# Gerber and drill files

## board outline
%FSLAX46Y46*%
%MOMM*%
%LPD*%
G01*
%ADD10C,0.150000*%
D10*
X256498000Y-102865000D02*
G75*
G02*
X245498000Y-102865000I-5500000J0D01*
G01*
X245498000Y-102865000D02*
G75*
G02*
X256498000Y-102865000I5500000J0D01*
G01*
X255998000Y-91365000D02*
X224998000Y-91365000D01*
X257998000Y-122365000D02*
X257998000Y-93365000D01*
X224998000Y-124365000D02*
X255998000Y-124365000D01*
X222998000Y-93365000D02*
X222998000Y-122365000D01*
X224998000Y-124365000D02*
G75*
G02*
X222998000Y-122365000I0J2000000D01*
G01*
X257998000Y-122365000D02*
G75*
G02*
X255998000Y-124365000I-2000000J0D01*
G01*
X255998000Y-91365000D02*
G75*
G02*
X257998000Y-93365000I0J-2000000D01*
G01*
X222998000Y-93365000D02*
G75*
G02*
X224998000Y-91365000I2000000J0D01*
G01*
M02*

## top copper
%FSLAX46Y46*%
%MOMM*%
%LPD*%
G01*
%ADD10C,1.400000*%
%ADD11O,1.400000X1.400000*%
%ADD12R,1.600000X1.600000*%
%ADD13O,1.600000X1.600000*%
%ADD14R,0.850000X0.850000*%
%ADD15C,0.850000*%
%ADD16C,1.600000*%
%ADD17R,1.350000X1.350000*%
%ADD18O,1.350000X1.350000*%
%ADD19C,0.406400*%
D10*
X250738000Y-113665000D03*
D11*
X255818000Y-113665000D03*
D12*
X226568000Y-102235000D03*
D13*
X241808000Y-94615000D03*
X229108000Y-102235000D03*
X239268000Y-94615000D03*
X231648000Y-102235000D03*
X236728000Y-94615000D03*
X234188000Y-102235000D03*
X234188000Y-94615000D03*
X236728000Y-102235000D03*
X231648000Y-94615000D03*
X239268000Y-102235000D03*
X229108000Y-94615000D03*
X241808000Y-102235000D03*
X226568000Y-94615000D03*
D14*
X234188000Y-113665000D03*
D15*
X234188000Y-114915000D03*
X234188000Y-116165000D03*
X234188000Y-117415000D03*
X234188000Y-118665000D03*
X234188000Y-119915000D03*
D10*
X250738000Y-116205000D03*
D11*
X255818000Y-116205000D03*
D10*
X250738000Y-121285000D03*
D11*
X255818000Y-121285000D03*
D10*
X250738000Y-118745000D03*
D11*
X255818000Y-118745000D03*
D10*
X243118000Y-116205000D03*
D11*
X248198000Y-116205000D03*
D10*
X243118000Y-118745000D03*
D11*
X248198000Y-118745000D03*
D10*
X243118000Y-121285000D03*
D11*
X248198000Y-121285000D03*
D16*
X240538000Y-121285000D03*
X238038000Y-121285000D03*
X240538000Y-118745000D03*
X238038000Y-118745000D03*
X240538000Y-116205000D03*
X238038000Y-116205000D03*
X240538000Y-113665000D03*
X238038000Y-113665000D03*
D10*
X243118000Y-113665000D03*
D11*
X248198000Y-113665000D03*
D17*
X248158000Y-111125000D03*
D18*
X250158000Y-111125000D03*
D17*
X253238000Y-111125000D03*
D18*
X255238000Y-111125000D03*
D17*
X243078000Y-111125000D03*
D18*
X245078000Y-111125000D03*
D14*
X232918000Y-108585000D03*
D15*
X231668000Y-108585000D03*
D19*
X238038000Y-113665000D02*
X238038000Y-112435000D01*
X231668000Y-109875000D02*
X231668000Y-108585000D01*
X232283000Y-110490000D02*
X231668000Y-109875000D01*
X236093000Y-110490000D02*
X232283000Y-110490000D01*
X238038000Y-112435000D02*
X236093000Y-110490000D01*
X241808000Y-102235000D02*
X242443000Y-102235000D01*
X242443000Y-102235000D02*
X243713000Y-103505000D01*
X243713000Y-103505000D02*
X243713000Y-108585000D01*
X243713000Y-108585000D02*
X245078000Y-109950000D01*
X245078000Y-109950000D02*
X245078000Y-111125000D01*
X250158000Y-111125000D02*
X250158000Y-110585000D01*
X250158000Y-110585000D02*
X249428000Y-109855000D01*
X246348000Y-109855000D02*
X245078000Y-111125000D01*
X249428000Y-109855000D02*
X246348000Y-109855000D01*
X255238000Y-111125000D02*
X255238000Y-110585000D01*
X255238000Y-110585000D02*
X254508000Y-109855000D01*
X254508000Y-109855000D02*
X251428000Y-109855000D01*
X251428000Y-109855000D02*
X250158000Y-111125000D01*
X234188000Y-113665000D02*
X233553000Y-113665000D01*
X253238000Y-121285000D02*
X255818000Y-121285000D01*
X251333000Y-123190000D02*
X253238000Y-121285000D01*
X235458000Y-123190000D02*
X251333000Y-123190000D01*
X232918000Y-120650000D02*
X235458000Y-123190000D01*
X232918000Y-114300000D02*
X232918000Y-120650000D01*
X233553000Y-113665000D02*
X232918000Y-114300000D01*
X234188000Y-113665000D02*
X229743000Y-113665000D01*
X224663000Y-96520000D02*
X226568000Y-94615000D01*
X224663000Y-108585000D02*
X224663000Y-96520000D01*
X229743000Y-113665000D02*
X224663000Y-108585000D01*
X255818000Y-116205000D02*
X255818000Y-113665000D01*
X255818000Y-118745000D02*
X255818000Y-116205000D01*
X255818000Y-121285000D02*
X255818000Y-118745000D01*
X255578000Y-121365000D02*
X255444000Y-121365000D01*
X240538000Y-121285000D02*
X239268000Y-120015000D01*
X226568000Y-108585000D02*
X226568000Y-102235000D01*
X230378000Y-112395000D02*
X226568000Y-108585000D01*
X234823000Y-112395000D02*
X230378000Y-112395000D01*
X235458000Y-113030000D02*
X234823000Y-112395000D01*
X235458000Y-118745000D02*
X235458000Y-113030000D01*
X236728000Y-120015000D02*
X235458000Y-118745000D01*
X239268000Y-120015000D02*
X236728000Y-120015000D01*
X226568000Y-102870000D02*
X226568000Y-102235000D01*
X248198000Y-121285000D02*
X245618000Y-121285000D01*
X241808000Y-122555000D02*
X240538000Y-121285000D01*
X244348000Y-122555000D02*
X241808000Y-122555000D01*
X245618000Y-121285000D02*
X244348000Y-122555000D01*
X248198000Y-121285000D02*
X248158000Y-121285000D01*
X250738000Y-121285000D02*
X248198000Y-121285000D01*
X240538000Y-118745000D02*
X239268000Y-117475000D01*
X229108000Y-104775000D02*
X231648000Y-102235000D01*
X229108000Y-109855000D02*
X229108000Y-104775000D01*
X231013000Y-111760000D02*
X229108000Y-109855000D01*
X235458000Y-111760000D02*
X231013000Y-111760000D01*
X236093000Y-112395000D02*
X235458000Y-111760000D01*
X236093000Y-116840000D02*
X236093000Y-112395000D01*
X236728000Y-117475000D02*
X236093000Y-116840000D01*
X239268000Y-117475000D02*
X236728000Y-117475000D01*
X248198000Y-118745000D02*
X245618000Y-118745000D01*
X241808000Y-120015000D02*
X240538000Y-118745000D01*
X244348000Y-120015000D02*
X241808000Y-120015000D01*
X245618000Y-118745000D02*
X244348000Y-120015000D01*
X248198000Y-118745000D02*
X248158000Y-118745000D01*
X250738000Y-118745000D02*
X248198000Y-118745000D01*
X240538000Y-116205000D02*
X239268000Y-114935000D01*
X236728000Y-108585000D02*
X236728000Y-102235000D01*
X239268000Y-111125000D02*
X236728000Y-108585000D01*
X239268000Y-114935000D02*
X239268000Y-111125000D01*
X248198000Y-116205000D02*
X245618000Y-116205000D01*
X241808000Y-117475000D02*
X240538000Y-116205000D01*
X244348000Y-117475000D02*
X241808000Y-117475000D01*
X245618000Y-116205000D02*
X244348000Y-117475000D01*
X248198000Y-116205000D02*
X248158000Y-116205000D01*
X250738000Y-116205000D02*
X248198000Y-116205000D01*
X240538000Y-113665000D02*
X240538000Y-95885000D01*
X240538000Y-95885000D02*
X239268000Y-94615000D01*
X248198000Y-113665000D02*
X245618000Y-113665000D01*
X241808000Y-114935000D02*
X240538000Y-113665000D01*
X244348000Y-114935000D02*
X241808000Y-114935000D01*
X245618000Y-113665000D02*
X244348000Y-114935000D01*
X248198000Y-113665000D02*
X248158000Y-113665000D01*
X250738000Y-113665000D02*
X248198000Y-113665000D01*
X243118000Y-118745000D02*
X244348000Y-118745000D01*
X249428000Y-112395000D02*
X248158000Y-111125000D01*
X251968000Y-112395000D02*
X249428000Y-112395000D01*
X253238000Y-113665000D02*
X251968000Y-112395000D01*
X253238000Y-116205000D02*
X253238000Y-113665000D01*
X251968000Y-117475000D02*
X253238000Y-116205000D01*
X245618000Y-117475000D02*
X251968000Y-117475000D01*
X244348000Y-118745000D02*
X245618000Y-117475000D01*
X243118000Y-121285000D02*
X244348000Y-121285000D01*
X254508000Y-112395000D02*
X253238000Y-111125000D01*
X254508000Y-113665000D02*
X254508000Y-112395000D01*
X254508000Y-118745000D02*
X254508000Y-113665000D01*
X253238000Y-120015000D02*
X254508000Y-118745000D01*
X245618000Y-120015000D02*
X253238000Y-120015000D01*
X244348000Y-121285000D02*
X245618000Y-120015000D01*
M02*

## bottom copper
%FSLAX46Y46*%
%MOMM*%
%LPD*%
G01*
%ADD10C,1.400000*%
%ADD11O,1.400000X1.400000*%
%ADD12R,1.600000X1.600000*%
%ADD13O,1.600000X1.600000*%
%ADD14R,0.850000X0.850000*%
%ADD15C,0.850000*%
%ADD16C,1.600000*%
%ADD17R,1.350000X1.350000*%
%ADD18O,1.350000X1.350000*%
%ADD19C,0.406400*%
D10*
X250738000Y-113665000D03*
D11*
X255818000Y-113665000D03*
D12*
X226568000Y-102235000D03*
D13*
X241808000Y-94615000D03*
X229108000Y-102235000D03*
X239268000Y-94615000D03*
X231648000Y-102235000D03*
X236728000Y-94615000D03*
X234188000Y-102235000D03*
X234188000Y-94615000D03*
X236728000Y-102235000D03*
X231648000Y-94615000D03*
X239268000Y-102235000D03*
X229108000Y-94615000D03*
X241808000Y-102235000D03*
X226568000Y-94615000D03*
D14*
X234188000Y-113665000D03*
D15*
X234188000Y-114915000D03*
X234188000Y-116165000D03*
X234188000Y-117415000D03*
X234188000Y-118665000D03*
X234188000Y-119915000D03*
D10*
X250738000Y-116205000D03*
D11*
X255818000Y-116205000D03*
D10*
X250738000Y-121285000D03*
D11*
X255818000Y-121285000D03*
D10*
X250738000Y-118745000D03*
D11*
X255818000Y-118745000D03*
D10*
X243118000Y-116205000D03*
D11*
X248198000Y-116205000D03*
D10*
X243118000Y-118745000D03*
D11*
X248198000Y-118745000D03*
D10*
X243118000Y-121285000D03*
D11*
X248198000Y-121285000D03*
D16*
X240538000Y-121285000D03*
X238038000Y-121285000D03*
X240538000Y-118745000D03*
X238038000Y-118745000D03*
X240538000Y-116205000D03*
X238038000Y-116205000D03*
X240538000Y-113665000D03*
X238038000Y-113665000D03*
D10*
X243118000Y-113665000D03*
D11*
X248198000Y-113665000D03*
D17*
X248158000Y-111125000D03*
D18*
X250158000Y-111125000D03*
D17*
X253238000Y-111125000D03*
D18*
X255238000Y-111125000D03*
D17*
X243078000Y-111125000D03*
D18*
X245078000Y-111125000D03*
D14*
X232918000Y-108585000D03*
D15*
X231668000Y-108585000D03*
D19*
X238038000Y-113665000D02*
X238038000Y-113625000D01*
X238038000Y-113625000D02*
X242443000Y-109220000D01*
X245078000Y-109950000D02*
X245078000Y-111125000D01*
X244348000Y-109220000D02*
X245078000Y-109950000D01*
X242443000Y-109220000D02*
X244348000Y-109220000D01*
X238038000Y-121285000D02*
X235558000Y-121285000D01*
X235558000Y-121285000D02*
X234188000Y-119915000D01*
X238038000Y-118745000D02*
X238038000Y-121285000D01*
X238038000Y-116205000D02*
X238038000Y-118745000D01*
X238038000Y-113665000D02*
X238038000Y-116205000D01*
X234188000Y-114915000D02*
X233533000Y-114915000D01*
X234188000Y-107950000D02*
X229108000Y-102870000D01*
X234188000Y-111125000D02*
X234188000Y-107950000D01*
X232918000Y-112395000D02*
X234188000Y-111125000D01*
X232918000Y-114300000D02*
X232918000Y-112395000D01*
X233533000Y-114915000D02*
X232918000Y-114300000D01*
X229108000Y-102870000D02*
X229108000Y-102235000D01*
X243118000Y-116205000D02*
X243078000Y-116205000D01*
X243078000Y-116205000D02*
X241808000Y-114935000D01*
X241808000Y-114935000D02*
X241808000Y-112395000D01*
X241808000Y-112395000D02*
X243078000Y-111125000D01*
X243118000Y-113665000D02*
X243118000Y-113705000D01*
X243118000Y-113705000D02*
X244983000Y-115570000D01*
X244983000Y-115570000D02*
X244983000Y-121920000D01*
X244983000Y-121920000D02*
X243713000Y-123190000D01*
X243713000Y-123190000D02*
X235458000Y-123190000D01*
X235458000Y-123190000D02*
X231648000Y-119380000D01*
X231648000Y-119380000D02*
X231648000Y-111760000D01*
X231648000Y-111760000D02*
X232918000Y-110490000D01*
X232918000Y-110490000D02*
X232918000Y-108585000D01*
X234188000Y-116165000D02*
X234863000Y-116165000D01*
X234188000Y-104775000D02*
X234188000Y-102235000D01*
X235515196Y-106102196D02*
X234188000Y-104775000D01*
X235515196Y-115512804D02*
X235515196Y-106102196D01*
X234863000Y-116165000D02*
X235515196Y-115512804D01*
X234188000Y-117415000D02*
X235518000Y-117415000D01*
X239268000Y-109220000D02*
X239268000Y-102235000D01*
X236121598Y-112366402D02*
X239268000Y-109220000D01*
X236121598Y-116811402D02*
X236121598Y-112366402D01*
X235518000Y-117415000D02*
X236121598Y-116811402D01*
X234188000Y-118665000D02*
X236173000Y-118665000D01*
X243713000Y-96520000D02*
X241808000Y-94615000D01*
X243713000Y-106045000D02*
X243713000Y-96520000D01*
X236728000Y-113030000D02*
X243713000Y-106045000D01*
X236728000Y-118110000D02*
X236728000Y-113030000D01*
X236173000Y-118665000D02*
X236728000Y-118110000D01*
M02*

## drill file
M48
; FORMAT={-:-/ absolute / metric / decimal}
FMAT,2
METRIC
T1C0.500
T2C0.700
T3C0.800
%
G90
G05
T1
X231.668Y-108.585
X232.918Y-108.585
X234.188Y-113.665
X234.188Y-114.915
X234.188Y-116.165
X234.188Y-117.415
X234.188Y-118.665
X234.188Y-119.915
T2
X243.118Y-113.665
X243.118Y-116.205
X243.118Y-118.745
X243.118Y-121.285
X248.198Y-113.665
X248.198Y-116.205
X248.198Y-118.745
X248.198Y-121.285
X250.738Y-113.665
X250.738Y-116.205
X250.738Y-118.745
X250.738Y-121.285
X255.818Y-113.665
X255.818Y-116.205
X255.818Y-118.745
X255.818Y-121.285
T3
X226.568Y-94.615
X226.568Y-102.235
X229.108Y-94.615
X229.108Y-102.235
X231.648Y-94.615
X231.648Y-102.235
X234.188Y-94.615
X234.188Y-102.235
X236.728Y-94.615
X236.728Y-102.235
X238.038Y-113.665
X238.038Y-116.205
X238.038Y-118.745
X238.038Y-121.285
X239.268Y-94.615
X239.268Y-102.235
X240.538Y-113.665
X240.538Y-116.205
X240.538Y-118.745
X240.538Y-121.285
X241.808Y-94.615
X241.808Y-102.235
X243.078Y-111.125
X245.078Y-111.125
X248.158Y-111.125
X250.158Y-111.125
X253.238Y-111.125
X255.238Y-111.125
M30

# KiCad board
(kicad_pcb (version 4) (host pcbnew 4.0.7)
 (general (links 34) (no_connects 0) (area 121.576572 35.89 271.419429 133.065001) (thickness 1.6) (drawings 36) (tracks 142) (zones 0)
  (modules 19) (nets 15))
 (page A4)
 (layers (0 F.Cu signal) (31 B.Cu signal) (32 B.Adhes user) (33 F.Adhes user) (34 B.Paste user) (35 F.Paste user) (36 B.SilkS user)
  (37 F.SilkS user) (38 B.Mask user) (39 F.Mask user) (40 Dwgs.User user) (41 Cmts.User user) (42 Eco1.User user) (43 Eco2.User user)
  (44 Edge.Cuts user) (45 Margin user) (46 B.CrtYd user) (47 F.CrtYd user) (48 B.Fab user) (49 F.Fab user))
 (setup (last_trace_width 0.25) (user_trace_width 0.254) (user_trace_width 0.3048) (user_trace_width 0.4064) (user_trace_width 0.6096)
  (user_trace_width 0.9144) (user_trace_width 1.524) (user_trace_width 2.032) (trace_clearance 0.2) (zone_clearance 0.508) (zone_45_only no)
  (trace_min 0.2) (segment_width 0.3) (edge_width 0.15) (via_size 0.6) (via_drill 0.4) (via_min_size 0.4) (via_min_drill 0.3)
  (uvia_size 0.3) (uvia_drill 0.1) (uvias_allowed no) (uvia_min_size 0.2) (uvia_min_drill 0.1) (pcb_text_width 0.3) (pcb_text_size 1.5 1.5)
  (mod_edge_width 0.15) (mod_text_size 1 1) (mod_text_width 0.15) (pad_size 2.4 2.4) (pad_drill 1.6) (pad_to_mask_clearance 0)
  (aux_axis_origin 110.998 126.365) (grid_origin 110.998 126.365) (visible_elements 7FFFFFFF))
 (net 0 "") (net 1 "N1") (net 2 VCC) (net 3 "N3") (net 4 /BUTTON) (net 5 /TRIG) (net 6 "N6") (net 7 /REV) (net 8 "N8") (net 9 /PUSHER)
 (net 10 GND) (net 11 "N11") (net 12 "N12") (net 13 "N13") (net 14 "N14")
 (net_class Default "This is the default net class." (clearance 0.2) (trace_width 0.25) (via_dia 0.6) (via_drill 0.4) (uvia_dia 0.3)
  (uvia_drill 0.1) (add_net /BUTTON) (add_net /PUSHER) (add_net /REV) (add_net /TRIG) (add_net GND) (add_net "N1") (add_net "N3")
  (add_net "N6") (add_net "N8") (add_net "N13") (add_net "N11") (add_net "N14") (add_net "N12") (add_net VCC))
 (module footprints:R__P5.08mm (layer F.Cu) (at 253.238 113.665)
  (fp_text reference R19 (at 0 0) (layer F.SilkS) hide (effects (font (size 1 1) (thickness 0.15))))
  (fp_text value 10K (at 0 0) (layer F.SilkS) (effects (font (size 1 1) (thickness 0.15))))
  (pad 1 thru_hole circle (at -2.5 0) (size 1.4 1.4) (drill 0.7) (layers *.Cu *.Mask) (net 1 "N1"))
  (pad 2 thru_hole oval (at 2.58 0) (size 1.4 1.4) (drill 0.7) (layers *.Cu *.Mask) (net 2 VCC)))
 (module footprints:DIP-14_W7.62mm (layer F.Cu) (at 226.568 102.235 90)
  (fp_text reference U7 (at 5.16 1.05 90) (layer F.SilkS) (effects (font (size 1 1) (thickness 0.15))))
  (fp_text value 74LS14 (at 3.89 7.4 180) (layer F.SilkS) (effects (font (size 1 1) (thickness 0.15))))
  (pad 1 thru_hole rect (at 0 0 90) (size 1.6 1.6) (drill 0.8) (layers *.Cu *.Mask) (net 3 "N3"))
  (pad 8 thru_hole oval (at 7.62 15.24 90) (size 1.6 1.6) (drill 0.8) (layers *.Cu *.Mask) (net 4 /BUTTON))
  (pad 2 thru_hole oval (at 0 2.54 90) (size 1.6 1.6) (drill 0.8) (layers *.Cu *.Mask) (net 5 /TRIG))
  (pad 9 thru_hole oval (at 7.62 12.7 90) (size 1.6 1.6) (drill 0.8) (layers *.Cu *.Mask) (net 1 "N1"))
  (pad 3 thru_hole oval (at 0 5.08 90) (size 1.6 1.6) (drill 0.8) (layers *.Cu *.Mask) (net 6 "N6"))
  (pad 10 thru_hole oval (at 7.62 10.16 90) (size 1.6 1.6) (drill 0.8) (layers *.Cu *.Mask))
  (pad 4 thru_hole oval (at 0 7.62 90) (size 1.6 1.6) (drill 0.8) (layers *.Cu *.Mask) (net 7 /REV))
  (pad 11 thru_hole oval (at 7.62 7.62 90) (size 1.6 1.6) (drill 0.8) (layers *.Cu *.Mask))
  (pad 5 thru_hole oval (at 0 10.16 90) (size 1.6 1.6) (drill 0.8) (layers *.Cu *.Mask) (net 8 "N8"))
  (pad 12 thru_hole oval (at 7.62 5.08 90) (size 1.6 1.6) (drill 0.8) (layers *.Cu *.Mask))
  (pad 6 thru_hole oval (at 0 12.7 90) (size 1.6 1.6) (drill 0.8) (layers *.Cu *.Mask) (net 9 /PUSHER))
  (pad 13 thru_hole oval (at 7.62 2.54 90) (size 1.6 1.6) (drill 0.8) (layers *.Cu *.Mask))
  (pad 7 thru_hole oval (at 0 15.24 90) (size 1.6 1.6) (drill 0.8) (layers *.Cu *.Mask) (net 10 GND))
  (pad 14 thru_hole oval (at 7.62 0 90) (size 1.6 1.6) (drill 0.8) (layers *.Cu *.Mask) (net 2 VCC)))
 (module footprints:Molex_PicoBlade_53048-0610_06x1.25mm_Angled (layer F.Cu) (at 234.188 113.665 270)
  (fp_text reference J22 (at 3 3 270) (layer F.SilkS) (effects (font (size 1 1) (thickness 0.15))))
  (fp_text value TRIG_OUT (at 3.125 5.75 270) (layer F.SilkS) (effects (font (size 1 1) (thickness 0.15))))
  (pad 1 thru_hole rect (at 0 0 270) (size 0.85 0.85) (drill 0.5) (layers *.Cu *.Mask) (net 2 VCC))
  (pad 2 thru_hole circle (at 1.25 0 270) (size 0.85 0.85) (drill 0.5) (layers *.Cu *.Mask) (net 5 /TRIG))
  (pad 3 thru_hole circle (at 2.5 0 270) (size 0.85 0.85) (drill 0.5) (layers *.Cu *.Mask) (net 7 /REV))
  (pad 4 thru_hole circle (at 3.75 0 270) (size 0.85 0.85) (drill 0.5) (layers *.Cu *.Mask) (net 9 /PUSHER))
  (pad 5 thru_hole circle (at 5 0 270) (size 0.85 0.85) (drill 0.5) (layers *.Cu *.Mask) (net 4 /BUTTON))
  (pad 6 thru_hole circle (at 6.25 0 270) (size 0.85 0.85) (drill 0.5) (layers *.Cu *.Mask) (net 10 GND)))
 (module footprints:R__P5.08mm (layer F.Cu) (at 253.238 116.205)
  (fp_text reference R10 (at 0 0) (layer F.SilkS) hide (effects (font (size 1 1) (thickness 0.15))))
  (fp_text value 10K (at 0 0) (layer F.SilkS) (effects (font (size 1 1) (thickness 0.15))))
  (pad 1 thru_hole circle (at -2.5 0) (size 1.4 1.4) (drill 0.7) (layers *.Cu *.Mask) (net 8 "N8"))
  (pad 2 thru_hole oval (at 2.58 0) (size 1.4 1.4) (drill 0.7) (layers *.Cu *.Mask) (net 2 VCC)))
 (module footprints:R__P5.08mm (layer F.Cu) (at 253.238 121.285)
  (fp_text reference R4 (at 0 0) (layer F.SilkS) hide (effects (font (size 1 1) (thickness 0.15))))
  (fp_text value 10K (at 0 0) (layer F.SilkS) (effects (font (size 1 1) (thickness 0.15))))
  (pad 1 thru_hole circle (at -2.5 0) (size 1.4 1.4) (drill 0.7) (layers *.Cu *.Mask) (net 3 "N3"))
  (pad 2 thru_hole oval (at 2.58 0) (size 1.4 1.4) (drill 0.7) (layers *.Cu *.Mask) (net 2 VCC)))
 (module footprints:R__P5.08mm (layer F.Cu) (at 253.238 118.745)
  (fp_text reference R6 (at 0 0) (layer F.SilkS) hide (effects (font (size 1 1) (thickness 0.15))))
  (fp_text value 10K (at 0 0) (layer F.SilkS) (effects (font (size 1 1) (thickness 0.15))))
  (pad 1 thru_hole circle (at -2.5 0) (size 1.4 1.4) (drill 0.7) (layers *.Cu *.Mask) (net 6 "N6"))
  (pad 2 thru_hole oval (at 2.58 0) (size 1.4 1.4) (drill 0.7) (layers *.Cu *.Mask) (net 2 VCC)))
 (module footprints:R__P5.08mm (layer F.Cu) (at 245.618 116.205)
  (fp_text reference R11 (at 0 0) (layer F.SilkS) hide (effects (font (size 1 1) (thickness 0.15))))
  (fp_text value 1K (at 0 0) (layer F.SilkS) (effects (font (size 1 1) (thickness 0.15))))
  (pad 1 thru_hole circle (at -2.5 0) (size 1.4 1.4) (drill 0.7) (layers *.Cu *.Mask) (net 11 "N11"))
  (pad 2 thru_hole oval (at 2.58 0) (size 1.4 1.4) (drill 0.7) (layers *.Cu *.Mask) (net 8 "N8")))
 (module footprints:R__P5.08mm (layer F.Cu) (at 245.618 118.745)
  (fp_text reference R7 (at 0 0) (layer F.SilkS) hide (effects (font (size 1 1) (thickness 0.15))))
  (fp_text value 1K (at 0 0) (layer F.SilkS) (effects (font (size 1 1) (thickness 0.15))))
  (pad 1 thru_hole circle (at -2.5 0) (size 1.4 1.4) (drill 0.7) (layers *.Cu *.Mask) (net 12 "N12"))
  (pad 2 thru_hole oval (at 2.58 0) (size 1.4 1.4) (drill 0.7) (layers *.Cu *.Mask) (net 6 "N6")))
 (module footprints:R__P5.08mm (layer F.Cu) (at 245.618 121.285)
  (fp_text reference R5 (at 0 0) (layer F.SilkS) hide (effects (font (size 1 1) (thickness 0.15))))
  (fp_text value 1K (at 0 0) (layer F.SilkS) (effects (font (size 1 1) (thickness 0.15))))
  (pad 1 thru_hole circle (at -2.5 0) (size 1.4 1.4) (drill 0.7) (layers *.Cu *.Mask) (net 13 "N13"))
  (pad 2 thru_hole oval (at 2.58 0) (size 1.4 1.4) (drill 0.7) (layers *.Cu *.Mask) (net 3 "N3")))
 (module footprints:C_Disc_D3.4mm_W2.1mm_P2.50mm (layer F.Cu) (at 240.538 121.285 180)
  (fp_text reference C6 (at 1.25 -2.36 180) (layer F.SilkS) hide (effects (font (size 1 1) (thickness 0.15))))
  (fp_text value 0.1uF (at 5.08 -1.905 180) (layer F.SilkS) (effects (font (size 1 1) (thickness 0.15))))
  (pad 1 thru_hole circle (at 0 0 180) (size 1.6 1.6) (drill 0.8) (layers *.Cu *.Mask) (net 3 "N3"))
  (pad 2 thru_hole circle (at 2.5 0 180) (size 1.6 1.6) (drill 0.8) (layers *.Cu *.Mask) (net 10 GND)))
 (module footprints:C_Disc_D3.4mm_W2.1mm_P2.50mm (layer F.Cu) (at 240.538 118.745 180)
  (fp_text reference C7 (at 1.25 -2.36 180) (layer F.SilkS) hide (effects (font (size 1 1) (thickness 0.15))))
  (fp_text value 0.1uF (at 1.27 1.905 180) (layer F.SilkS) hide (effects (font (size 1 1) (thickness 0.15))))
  (pad 1 thru_hole circle (at 0 0 180) (size 1.6 1.6) (drill 0.8) (layers *.Cu *.Mask) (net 6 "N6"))
  (pad 2 thru_hole circle (at 2.5 0 180) (size 1.6 1.6) (drill 0.8) (layers *.Cu *.Mask) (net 10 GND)))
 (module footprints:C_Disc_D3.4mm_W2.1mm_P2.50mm (layer F.Cu) (at 240.538 116.205 180)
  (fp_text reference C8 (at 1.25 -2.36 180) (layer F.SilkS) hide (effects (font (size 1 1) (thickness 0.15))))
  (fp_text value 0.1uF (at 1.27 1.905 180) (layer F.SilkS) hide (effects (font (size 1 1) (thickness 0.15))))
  (pad 1 thru_hole circle (at 0 0 180) (size 1.6 1.6) (drill 0.8) (layers *.Cu *.Mask) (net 8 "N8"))
  (pad 2 thru_hole circle (at 2.5 0 180) (size 1.6 1.6) (drill 0.8) (layers *.Cu *.Mask) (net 10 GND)))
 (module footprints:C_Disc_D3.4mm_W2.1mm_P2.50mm (layer F.Cu) (at 240.538 113.665 180)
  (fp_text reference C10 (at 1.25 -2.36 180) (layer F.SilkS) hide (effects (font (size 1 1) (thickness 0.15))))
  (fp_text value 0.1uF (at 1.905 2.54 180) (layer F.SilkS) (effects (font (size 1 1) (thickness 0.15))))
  (pad 1 thru_hole circle (at 0 0 180) (size 1.6 1.6) (drill 0.8) (layers *.Cu *.Mask) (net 1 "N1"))
  (pad 2 thru_hole circle (at 2.5 0 180) (size 1.6 1.6) (drill 0.8) (layers *.Cu *.Mask) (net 10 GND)))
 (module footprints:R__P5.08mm (layer F.Cu) (at 245.618 113.665)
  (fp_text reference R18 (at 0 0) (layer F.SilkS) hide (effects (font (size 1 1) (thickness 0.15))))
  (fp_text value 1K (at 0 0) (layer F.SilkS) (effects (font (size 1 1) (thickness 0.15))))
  (pad 1 thru_hole circle (at -2.5 0) (size 1.4 1.4) (drill 0.7) (layers *.Cu *.Mask) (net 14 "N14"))
  (pad 2 thru_hole oval (at 2.58 0) (size 1.4 1.4) (drill 0.7) (layers *.Cu *.Mask) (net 1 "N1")))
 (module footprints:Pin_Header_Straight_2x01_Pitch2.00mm (layer F.Cu) (at 248.158 111.125)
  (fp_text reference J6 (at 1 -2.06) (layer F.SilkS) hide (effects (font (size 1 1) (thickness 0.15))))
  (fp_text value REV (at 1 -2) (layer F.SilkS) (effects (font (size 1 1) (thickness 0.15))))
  (pad 1 thru_hole rect (at 0 0) (size 1.35 1.35) (drill 0.8) (layers *.Cu *.Mask) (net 12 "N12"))
  (pad 2 thru_hole oval (at 2 0) (size 1.35 1.35) (drill 0.8) (layers *.Cu *.Mask) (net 10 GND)))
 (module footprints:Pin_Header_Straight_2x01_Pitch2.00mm (layer F.Cu) (at 253.238 111.125)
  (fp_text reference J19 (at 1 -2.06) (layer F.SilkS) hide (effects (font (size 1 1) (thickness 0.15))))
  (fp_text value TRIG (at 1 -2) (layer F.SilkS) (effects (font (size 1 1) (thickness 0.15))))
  (pad 1 thru_hole rect (at 0 0) (size 1.35 1.35) (drill 0.8) (layers *.Cu *.Mask) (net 13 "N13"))
  (pad 2 thru_hole oval (at 2 0) (size 1.35 1.35) (drill 0.8) (layers *.Cu *.Mask) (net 10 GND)))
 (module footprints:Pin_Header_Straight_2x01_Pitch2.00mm (layer F.Cu) (at 243.078 111.125)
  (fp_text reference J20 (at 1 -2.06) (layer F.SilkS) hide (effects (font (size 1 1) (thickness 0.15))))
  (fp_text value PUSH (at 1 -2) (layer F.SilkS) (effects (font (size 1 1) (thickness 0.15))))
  (pad 1 thru_hole rect (at 0 0) (size 1.35 1.35) (drill 0.8) (layers *.Cu *.Mask) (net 11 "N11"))
  (pad 2 thru_hole oval (at 2 0) (size 1.35 1.35) (drill 0.8) (layers *.Cu *.Mask) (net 10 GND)))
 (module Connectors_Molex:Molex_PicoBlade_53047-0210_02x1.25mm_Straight (layer F.Cu) (at 232.918 108.585 180)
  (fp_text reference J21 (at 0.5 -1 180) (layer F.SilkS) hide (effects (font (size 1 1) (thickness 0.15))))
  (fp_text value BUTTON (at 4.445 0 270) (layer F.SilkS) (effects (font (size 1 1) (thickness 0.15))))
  (pad 1 thru_hole rect (at 0 0 180) (size 0.85 0.85) (drill 0.5) (layers *.Cu *.Mask) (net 14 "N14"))
  (pad 2 thru_hole circle (at 1.25 0 180) (size 0.85 0.85) (drill 0.5) (layers *.Cu *.Mask) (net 10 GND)))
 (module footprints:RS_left (layer F.Cu) (at 237.998 105.41)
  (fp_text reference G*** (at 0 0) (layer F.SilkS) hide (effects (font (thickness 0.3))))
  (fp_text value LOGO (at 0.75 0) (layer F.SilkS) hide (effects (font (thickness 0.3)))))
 (gr_circle (center 250.998 102.865) (end 245.498 102.865) (layer Edge.Cuts) (width 0.15))
 (gr_line (start 255.998 91.365) (end 224.998 91.365) (angle 90) (layer Edge.Cuts) (width 0.15))
 (gr_line (start 257.998 122.365) (end 257.998 93.365) (angle 90) (layer Edge.Cuts) (width 0.15))
 (gr_line (start 224.998 124.365) (end 255.998 124.365) (angle 90) (layer Edge.Cuts) (width 0.15))
 (gr_line (start 222.998 93.365) (end 222.998 122.365) (angle 90) (layer Edge.Cuts) (width 0.15))
 (gr_arc (start 224.998 122.365) (end 224.998 124.365) (angle 90) (layer Edge.Cuts) (width 0.15))
 (gr_arc (start 255.998 122.365) (end 257.998 122.365) (angle 90) (layer Edge.Cuts) (width 0.15))
 (gr_arc (start 255.998 93.365) (end 255.998 91.365) (angle 90) (layer Edge.Cuts) (width 0.15))
 (gr_arc (start 224.998 93.365) (end 222.998 93.365) (angle 90) (layer Edge.Cuts) (width 0.15))
 (segment (start 238.038 113.665) (end 238.038 113.625) (width 0.4064) (layer B.Cu) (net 10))
 (segment (start 238.038 113.625) (end 242.443 109.22) (width 0.4064) (layer B.Cu) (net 10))
 (segment (start 245.078 109.95) (end 245.078 111.125) (width 0.4064) (layer B.Cu) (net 10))
 (segment (start 244.348 109.22) (end 245.078 109.95) (width 0.4064) (layer B.Cu) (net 10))
 (segment (start 242.443 109.22) (end 244.348 109.22) (width 0.4064) (layer B.Cu) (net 10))
 (segment (start 238.038 113.665) (end 238.038 112.435) (width 0.4064) (layer F.Cu) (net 10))
 (segment (start 231.668 109.875) (end 231.668 108.585) (width 0.4064) (layer F.Cu) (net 10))
 (segment (start 232.283 110.49) (end 231.668 109.875) (width 0.4064) (layer F.Cu) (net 10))
 (segment (start 236.093 110.49) (end 232.283 110.49) (width 0.4064) (layer F.Cu) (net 10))
 (segment (start 238.038 112.435) (end 236.093 110.49) (width 0.4064) (layer F.Cu) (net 10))
 (segment (start 241.808 102.235) (end 242.443 102.235) (width 0.4064) (layer F.Cu) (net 10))
 (segment (start 242.443 102.235) (end 243.713 103.505) (width 0.4064) (layer F.Cu) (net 10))
 (segment (start 243.713 103.505) (end 243.713 108.585) (width 0.4064) (layer F.Cu) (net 10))
 (segment (start 243.713 108.585) (end 245.078 109.95) (width 0.4064) (layer F.Cu) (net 10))
 (segment (start 245.078 109.95) (end 245.078 111.125) (width 0.4064) (layer F.Cu) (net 10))
 (segment (start 250.158 111.125) (end 250.158 110.585) (width 0.4064) (layer F.Cu) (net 10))
 (segment (start 250.158 110.585) (end 249.428 109.855) (width 0.4064) (layer F.Cu) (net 10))
 (segment (start 246.348 109.855) (end 245.078 111.125) (width 0.4064) (layer F.Cu) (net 10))
 (segment (start 249.428 109.855) (end 246.348 109.855) (width 0.4064) (layer F.Cu) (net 10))
 (segment (start 255.238 111.125) (end 255.238 110.585) (width 0.4064) (layer F.Cu) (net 10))
 (segment (start 255.238 110.585) (end 254.508 109.855) (width 0.4064) (layer F.Cu) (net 10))
 (segment (start 254.508 109.855) (end 251.428 109.855) (width 0.4064) (layer F.Cu) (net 10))
 (segment (start 251.428 109.855) (end 250.158 111.125) (width 0.4064) (layer F.Cu) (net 10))
 (segment (start 238.038 121.285) (end 235.558 121.285) (width 0.4064) (layer B.Cu) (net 10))
 (segment (start 235.558 121.285) (end 234.188 119.915) (width 0.4064) (layer B.Cu) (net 10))
 (segment (start 238.038 118.745) (end 238.038 121.285) (width 0.4064) (layer B.Cu) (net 10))
 (segment (start 238.038 116.205) (end 238.038 118.745) (width 0.4064) (layer B.Cu) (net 10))
 (segment (start 238.038 113.665) (end 238.038 116.205) (width 0.4064) (layer B.Cu) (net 10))
 (segment (start 234.188 113.665) (end 233.553 113.665) (width 0.4064) (layer F.Cu) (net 2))
 (segment (start 253.238 121.285) (end 255.818 121.285) (width 0.4064) (layer F.Cu) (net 2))
 (segment (start 251.333 123.19) (end 253.238 121.285) (width 0.4064) (layer F.Cu) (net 2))
 (segment (start 235.458 123.19) (end 251.333 123.19) (width 0.4064) (layer F.Cu) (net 2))
 (segment (start 232.918 120.65) (end 235.458 123.19) (width 0.4064) (layer F.Cu) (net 2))
 (segment (start 232.918 114.3) (end 232.918 120.65) (width 0.4064) (layer F.Cu) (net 2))
 (segment (start 233.553 113.665) (end 232.918 114.3) (width 0.4064) (layer F.Cu) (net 2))
 (segment (start 234.188 113.665) (end 229.743 113.665) (width 0.4064) (layer F.Cu) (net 2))
 (segment (start 224.663 96.52) (end 226.568 94.615) (width 0.4064) (layer F.Cu) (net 2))
 (segment (start 224.663 108.585) (end 224.663 96.52) (width 0.4064) (layer F.Cu) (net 2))
 (segment (start 229.743 113.665) (end 224.663 108.585) (width 0.4064) (layer F.Cu) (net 2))
 (segment (start 255.818 116.205) (end 255.818 113.665) (width 0.4064) (layer F.Cu) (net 2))
 (segment (start 255.818 118.745) (end 255.818 116.205) (width 0.4064) (layer F.Cu) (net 2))
 (segment (start 255.818 121.285) (end 255.818 118.745) (width 0.4064) (layer F.Cu) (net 2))
 (segment (start 255.578 121.365) (end 255.444 121.365) (width 0.4064) (layer F.Cu) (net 2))
 (segment (start 234.188 114.915) (end 233.533 114.915) (width 0.4064) (layer B.Cu) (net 5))
 (segment (start 234.188 107.95) (end 229.108 102.87) (width 0.4064) (layer B.Cu) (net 5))
 (segment (start 234.188 111.125) (end 234.188 107.95) (width 0.4064) (layer B.Cu) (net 5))
 (segment (start 232.918 112.395) (end 234.188 111.125) (width 0.4064) (layer B.Cu) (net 5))
 (segment (start 232.918 114.3) (end 232.918 112.395) (width 0.4064) (layer B.Cu) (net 5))
 (segment (start 233.533 114.915) (end 232.918 114.3) (width 0.4064) (layer B.Cu) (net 5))
 (segment (start 229.108 102.87) (end 229.108 102.235) (width 0.4064) (layer B.Cu) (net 5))
 (segment (start 240.538 121.285) (end 239.268 120.015) (width 0.4064) (layer F.Cu) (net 3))
 (segment (start 226.568 108.585) (end 226.568 102.235) (width 0.4064) (layer F.Cu) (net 3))
 (segment (start 230.378 112.395) (end 226.568 108.585) (width 0.4064) (layer F.Cu) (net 3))
 (segment (start 234.823 112.395) (end 230.378 112.395) (width 0.4064) (layer F.Cu) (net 3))
 (segment (start 235.458 113.03) (end 234.823 112.395) (width 0.4064) (layer F.Cu) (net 3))
 (segment (start 235.458 118.745) (end 235.458 113.03) (width 0.4064) (layer F.Cu) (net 3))
 (segment (start 236.728 120.015) (end 235.458 118.745) (width 0.4064) (layer F.Cu) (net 3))
 (segment (start 239.268 120.015) (end 236.728 120.015) (width 0.4064) (layer F.Cu) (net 3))
 (segment (start 226.568 102.87) (end 226.568 102.235) (width 0.4064) (layer F.Cu) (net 3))
 (segment (start 248.198 121.285) (end 245.618 121.285) (width 0.4064) (layer F.Cu) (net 3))
 (segment (start 241.808 122.555) (end 240.538 121.285) (width 0.4064) (layer F.Cu) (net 3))
 (segment (start 244.348 122.555) (end 241.808 122.555) (width 0.4064) (layer F.Cu) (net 3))
 (segment (start 245.618 121.285) (end 244.348 122.555) (width 0.4064) (layer F.Cu) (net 3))
 (segment (start 248.198 121.285) (end 248.158 121.285) (width 0.4064) (layer F.Cu) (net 3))
 (segment (start 250.738 121.285) (end 248.198 121.285) (width 0.4064) (layer F.Cu) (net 3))
 (segment (start 240.538 118.745) (end 239.268 117.475) (width 0.4064) (layer F.Cu) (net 6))
 (segment (start 229.108 104.775) (end 231.648 102.235) (width 0.4064) (layer F.Cu) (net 6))
 (segment (start 229.108 109.855) (end 229.108 104.775) (width 0.4064) (layer F.Cu) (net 6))
 (segment (start 231.013 111.76) (end 229.108 109.855) (width 0.4064) (layer F.Cu) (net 6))
 (segment (start 235.458 111.76) (end 231.013 111.76) (width 0.4064) (layer F.Cu) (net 6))
 (segment (start 236.093 112.395) (end 235.458 111.76) (width 0.4064) (layer F.Cu) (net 6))
 (segment (start 236.093 116.84) (end 236.093 112.395) (width 0.4064) (layer F.Cu) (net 6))
 (segment (start 236.728 117.475) (end 236.093 116.84) (width 0.4064) (layer F.Cu) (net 6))
 (segment (start 239.268 117.475) (end 236.728 117.475) (width 0.4064) (layer F.Cu) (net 6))
 (segment (start 248.198 118.745) (end 245.618 118.745) (width 0.4064) (layer F.Cu) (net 6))
 (segment (start 241.808 120.015) (end 240.538 118.745) (width 0.4064) (layer F.Cu) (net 6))
 (segment (start 244.348 120.015) (end 241.808 120.015) (width 0.4064) (layer F.Cu) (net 6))
 (segment (start 245.618 118.745) (end 244.348 120.015) (width 0.4064) (layer F.Cu) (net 6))
 (segment (start 248.198 118.745) (end 248.158 118.745) (width 0.4064) (layer F.Cu) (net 6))
 (segment (start 250.738 118.745) (end 248.198 118.745) (width 0.4064) (layer F.Cu) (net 6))
 (segment (start 240.538 116.205) (end 239.268 114.935) (width 0.4064) (layer F.Cu) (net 8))
 (segment (start 236.728 108.585) (end 236.728 102.235) (width 0.4064) (layer F.Cu) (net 8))
 (segment (start 239.268 111.125) (end 236.728 108.585) (width 0.4064) (layer F.Cu) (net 8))
 (segment (start 239.268 114.935) (end 239.268 111.125) (width 0.4064) (layer F.Cu) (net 8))
 (segment (start 248.198 116.205) (end 245.618 116.205) (width 0.4064) (layer F.Cu) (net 8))
 (segment (start 241.808 117.475) (end 240.538 116.205) (width 0.4064) (layer F.Cu) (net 8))
 (segment (start 244.348 117.475) (end 241.808 117.475) (width 0.4064) (layer F.Cu) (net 8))
 (segment (start 245.618 116.205) (end 244.348 117.475) (width 0.4064) (layer F.Cu) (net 8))
 (segment (start 248.198 116.205) (end 248.158 116.205) (width 0.4064) (layer F.Cu) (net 8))
 (segment (start 250.738 116.205) (end 248.198 116.205) (width 0.4064) (layer F.Cu) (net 8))
 (segment (start 240.538 113.665) (end 240.538 95.885) (width 0.4064) (layer F.Cu) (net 1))
 (segment (start 240.538 95.885) (end 239.268 94.615) (width 0.4064) (layer F.Cu) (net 1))
 (segment (start 248.198 113.665) (end 245.618 113.665) (width 0.4064) (layer F.Cu) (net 1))
 (segment (start 241.808 114.935) (end 240.538 113.665) (width 0.4064) (layer F.Cu) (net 1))
 (segment (start 244.348 114.935) (end 241.808 114.935) (width 0.4064) (layer F.Cu) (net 1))
 (segment (start 245.618 113.665) (end 244.348 114.935) (width 0.4064) (layer F.Cu) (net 1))
 (segment (start 248.198 113.665) (end 248.158 113.665) (width 0.4064) (layer F.Cu) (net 1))
 (segment (start 250.738 113.665) (end 248.198 113.665) (width 0.4064) (layer F.Cu) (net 1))
 (segment (start 243.118 118.745) (end 244.348 118.745) (width 0.4064) (layer F.Cu) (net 12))
 (segment (start 249.428 112.395) (end 248.158 111.125) (width 0.4064) (layer F.Cu) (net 12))
 (segment (start 251.968 112.395) (end 249.428 112.395) (width 0.4064) (layer F.Cu) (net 12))
 (segment (start 253.238 113.665) (end 251.968 112.395) (width 0.4064) (layer F.Cu) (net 12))
 (segment (start 253.238 116.205) (end 253.238 113.665) (width 0.4064) (layer F.Cu) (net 12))
 (segment (start 251.968 117.475) (end 253.238 116.205) (width 0.4064) (layer F.Cu) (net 12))
 (segment (start 245.618 117.475) (end 251.968 117.475) (width 0.4064) (layer F.Cu) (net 12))
 (segment (start 244.348 118.745) (end 245.618 117.475) (width 0.4064) (layer F.Cu) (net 12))
 (segment (start 243.118 121.285) (end 244.348 121.285) (width 0.4064) (layer F.Cu) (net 13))
 (segment (start 254.508 112.395) (end 253.238 111.125) (width 0.4064) (layer F.Cu) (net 13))
 (segment (start 254.508 113.665) (end 254.508 112.395) (width 0.4064) (layer F.Cu) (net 13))
 (segment (start 254.508 118.745) (end 254.508 113.665) (width 0.4064) (layer F.Cu) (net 13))
 (segment (start 253.238 120.015) (end 254.508 118.745) (width 0.4064) (layer F.Cu) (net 13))
 (segment (start 245.618 120.015) (end 253.238 120.015) (width 0.4064) (layer F.Cu) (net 13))
 (segment (start 244.348 121.285) (end 245.618 120.015) (width 0.4064) (layer F.Cu) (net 13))
 (segment (start 243.118 116.205) (end 243.078 116.205) (width 0.4064) (layer B.Cu) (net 11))
 (segment (start 243.078 116.205) (end 241.808 114.935) (width 0.4064) (layer B.Cu) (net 11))
 (segment (start 241.808 114.935) (end 241.808 112.395) (width 0.4064) (layer B.Cu) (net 11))
 (segment (start 241.808 112.395) (end 243.078 111.125) (width 0.4064) (layer B.Cu) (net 11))
 (segment (start 243.118 113.665) (end 243.118 113.705) (width 0.4064) (layer B.Cu) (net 14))
 (segment (start 243.118 113.705) (end 244.983 115.57) (width 0.4064) (layer B.Cu) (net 14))
 (segment (start 244.983 115.57) (end 244.983 121.92) (width 0.4064) (layer B.Cu) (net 14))
 (segment (start 244.983 121.92) (end 243.713 123.19) (width 0.4064) (layer B.Cu) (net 14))
 (segment (start 243.713 123.19) (end 235.458 123.19) (width 0.4064) (layer B.Cu) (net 14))
 (segment (start 235.458 123.19) (end 231.648 119.38) (width 0.4064) (layer B.Cu) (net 14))
 (segment (start 231.648 119.38) (end 231.648 111.76) (width 0.4064) (layer B.Cu) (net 14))
 (segment (start 231.648 111.76) (end 232.918 110.49) (width 0.4064) (layer B.Cu) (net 14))
 (segment (start 232.918 110.49) (end 232.918 108.585) (width 0.4064) (layer B.Cu) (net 14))
 (segment (start 234.188 116.165) (end 234.863 116.165) (width 0.4064) (layer B.Cu) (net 7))
 (segment (start 234.188 104.775) (end 234.188 102.235) (width 0.4064) (layer B.Cu) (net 7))
 (segment (start 235.515196 106.102196) (end 234.188 104.775) (width 0.4064) (layer B.Cu) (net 7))
 (segment (start 235.515196 115.512804) (end 235.515196 106.102196) (width 0.4064) (layer B.Cu) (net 7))
 (segment (start 234.863 116.165) (end 235.515196 115.512804) (width 0.4064) (layer B.Cu) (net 7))
 (segment (start 234.188 117.415) (end 235.518 117.415) (width 0.4064) (layer B.Cu) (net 9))
 (segment (start 239.268 109.22) (end 239.268 102.235) (width 0.4064) (layer B.Cu) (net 9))
 (segment (start 236.121598 112.366402) (end 239.268 109.22) (width 0.4064) (layer B.Cu) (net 9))
 (segment (start 236.121598 116.811402) (end 236.121598 112.366402) (width 0.4064) (layer B.Cu) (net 9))
 (segment (start 235.518 117.415) (end 236.121598 116.811402) (width 0.4064) (layer B.Cu) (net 9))
 (segment (start 234.188 118.665) (end 236.173 118.665) (width 0.4064) (layer B.Cu) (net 4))
 (segment (start 243.713 96.52) (end 241.808 94.615) (width 0.4064) (layer B.Cu) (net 4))
 (segment (start 243.713 106.045) (end 243.713 96.52) (width 0.4064) (layer B.Cu) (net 4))
 (segment (start 236.728 113.03) (end 243.713 106.045) (width 0.4064) (layer B.Cu) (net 4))
 (segment (start 236.728 118.11) (end 236.728 113.03) (width 0.4064) (layer B.Cu) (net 4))
 (segment (start 236.173 118.665) (end 236.728 118.11) (width 0.4064) (layer B.Cu) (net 4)))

